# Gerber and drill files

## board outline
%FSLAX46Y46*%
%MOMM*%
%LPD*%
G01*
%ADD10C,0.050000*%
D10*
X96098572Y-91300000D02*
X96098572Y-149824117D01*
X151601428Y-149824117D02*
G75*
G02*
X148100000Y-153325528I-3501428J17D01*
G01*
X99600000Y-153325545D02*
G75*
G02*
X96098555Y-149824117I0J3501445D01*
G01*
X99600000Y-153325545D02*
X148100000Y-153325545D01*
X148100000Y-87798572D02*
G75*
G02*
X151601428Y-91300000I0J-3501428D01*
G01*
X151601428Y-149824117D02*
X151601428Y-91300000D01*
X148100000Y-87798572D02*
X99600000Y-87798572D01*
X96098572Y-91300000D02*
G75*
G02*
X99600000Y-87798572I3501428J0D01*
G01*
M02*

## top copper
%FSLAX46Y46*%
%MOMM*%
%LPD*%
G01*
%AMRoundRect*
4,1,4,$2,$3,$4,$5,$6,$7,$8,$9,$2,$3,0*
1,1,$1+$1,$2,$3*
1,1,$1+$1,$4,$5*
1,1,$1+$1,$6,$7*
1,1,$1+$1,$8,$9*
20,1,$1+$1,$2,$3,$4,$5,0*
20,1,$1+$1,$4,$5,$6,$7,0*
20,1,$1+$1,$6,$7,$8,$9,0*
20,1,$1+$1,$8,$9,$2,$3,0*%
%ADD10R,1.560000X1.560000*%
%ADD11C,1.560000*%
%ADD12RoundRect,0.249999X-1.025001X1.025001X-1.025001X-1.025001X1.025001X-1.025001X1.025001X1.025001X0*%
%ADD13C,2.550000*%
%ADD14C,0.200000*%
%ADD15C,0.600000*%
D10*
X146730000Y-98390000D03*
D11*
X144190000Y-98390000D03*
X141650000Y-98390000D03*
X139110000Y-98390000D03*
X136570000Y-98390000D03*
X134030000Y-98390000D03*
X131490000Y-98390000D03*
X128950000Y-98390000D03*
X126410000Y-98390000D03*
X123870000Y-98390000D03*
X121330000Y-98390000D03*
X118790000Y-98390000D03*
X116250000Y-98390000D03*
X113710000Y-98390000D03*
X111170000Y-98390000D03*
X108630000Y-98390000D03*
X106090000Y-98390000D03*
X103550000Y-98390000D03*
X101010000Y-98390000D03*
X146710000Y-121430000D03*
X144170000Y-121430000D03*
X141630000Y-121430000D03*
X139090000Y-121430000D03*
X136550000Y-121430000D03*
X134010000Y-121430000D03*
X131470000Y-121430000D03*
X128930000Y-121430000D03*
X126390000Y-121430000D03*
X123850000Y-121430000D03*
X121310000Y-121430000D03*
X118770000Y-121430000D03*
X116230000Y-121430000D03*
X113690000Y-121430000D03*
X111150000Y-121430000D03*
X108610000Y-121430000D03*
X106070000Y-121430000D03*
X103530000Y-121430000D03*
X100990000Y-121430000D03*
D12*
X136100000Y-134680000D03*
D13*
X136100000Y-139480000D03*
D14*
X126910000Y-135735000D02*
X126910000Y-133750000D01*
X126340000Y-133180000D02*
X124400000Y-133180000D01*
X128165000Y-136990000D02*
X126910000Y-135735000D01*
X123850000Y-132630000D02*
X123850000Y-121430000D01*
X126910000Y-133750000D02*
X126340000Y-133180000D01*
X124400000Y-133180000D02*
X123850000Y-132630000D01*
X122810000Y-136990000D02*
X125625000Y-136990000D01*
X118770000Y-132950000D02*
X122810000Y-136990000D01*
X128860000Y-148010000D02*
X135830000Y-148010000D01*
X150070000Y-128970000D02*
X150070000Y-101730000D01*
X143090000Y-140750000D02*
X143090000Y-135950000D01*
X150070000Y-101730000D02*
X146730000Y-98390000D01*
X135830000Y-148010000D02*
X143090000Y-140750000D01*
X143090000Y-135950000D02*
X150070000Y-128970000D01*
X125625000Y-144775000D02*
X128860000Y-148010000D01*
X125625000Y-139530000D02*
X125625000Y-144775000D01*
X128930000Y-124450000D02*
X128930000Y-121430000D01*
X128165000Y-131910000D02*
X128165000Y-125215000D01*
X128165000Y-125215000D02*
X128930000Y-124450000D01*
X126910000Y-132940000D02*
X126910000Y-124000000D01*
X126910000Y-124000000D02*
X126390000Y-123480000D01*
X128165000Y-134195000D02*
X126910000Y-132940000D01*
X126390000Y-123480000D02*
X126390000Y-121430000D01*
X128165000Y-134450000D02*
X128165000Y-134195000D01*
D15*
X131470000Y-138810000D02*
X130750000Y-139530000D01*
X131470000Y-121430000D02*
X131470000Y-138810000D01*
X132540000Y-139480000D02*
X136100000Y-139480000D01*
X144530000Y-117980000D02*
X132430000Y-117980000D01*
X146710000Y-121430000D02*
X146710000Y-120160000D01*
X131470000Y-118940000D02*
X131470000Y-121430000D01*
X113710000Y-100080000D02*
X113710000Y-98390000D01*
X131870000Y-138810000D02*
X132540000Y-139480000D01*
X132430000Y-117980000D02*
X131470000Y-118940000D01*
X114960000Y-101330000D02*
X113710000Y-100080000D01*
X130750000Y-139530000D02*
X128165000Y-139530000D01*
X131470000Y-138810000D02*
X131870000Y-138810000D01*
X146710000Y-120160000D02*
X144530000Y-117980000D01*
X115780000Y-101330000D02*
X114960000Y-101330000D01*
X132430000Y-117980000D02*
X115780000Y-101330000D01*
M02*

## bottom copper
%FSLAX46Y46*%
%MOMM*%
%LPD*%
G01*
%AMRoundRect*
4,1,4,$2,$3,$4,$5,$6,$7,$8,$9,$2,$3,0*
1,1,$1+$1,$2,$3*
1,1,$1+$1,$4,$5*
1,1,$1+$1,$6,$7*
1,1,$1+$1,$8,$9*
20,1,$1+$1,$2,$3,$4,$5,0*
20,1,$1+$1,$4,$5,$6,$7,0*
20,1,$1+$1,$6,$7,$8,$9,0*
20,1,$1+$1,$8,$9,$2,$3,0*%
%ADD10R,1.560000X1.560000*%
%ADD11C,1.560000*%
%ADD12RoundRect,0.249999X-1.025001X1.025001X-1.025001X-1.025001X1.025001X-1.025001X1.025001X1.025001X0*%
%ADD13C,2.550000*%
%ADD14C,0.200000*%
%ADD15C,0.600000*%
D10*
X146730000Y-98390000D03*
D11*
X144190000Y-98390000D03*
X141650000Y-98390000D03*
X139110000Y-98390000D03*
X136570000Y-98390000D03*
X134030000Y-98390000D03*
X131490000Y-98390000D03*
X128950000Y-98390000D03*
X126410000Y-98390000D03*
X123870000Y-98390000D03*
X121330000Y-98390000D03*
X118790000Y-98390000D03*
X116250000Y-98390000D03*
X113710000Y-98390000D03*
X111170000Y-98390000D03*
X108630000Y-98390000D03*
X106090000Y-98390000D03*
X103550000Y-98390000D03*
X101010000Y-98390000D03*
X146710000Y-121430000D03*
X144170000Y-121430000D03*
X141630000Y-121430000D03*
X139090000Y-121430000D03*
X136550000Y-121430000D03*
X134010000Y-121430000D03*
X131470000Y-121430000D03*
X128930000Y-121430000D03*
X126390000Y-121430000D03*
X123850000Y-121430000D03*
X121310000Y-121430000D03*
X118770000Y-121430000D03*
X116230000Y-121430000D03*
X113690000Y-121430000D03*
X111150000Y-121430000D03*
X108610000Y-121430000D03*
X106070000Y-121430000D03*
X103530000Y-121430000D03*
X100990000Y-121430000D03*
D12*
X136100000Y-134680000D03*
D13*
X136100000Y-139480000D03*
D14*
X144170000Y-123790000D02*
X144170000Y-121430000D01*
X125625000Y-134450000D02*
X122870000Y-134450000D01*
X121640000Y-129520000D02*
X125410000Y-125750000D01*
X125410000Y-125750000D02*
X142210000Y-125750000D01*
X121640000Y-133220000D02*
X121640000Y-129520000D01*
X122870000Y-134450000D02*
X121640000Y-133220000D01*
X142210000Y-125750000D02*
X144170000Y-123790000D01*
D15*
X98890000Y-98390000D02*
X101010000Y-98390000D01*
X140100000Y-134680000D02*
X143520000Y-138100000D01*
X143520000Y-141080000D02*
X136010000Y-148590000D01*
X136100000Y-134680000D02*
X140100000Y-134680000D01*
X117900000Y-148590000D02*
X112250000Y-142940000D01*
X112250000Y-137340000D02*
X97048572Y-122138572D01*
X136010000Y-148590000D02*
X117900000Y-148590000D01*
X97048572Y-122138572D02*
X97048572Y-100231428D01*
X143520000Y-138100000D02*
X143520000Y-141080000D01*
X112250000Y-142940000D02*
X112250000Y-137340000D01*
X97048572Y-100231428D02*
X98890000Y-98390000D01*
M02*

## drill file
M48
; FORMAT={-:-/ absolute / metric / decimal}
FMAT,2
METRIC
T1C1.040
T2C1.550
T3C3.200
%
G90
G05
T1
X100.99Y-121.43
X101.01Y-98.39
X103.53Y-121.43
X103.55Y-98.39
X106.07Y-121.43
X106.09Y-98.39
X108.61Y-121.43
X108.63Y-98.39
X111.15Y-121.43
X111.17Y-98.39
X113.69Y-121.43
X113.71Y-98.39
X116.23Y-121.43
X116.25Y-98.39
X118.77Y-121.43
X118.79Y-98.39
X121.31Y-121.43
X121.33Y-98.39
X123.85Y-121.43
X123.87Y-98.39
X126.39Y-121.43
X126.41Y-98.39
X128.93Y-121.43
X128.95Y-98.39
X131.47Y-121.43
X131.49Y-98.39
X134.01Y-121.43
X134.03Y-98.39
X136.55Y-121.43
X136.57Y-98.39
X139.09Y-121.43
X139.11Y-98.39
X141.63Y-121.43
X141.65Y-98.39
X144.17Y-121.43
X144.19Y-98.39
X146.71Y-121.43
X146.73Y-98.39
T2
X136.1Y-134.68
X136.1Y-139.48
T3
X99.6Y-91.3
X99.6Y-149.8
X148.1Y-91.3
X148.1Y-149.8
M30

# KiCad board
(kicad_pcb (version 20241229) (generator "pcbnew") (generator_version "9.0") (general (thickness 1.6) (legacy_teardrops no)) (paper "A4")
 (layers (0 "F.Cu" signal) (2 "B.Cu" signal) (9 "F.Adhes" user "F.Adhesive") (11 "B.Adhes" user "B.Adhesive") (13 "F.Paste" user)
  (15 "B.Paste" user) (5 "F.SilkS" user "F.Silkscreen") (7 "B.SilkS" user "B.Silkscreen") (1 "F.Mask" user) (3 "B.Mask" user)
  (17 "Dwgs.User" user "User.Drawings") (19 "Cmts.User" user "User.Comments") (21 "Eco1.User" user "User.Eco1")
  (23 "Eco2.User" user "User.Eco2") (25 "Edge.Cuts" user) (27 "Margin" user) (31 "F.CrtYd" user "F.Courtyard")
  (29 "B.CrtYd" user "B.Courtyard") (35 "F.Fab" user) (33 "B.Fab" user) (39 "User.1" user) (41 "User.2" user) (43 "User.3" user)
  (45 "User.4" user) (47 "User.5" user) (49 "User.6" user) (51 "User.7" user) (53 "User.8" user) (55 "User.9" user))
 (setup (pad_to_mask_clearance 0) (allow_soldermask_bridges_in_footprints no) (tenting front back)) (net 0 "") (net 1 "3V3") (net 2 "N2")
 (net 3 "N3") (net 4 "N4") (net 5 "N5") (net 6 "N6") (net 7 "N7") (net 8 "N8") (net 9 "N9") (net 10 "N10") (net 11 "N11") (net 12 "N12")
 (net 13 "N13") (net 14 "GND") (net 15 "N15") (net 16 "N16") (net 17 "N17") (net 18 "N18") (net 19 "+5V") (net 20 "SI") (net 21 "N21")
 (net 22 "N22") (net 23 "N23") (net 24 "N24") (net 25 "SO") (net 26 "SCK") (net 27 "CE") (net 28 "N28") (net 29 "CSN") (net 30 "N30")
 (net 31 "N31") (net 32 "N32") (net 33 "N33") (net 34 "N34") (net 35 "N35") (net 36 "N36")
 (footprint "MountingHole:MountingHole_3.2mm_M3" (layer "F.Cu") (at 148.1 91.3 180)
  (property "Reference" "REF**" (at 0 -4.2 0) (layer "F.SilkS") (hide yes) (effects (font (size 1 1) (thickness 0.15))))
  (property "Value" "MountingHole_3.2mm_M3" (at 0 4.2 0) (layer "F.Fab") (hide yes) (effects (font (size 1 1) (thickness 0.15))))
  (pad "" np_thru_hole circle (at 0 0 180) (size 3.2 3.2) (drill 3.2) (layers "*.Cu" "*.Mask")))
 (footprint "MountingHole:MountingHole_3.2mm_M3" (layer "F.Cu") (at 99.6 91.3 180)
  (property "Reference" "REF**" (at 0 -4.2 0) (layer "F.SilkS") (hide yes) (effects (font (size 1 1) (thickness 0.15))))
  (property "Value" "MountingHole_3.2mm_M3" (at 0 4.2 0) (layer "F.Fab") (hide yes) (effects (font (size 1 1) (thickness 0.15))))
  (pad "" np_thru_hole circle (at 0 0 180) (size 3.2 3.2) (drill 3.2) (layers "*.Cu" "*.Mask")))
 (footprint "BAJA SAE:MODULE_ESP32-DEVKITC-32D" (layer "F.Cu") (at 127.8 110.15 -90)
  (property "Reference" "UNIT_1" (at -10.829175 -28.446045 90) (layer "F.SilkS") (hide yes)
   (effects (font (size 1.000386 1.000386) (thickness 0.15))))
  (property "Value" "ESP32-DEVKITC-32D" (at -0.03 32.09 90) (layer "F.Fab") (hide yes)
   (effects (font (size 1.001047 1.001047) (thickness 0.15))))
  (pad "J2-1" thru_hole rect (at -11.76 -18.93 270) (size 1.56 1.56) (drill 1.04) (layers "*.Cu" "*.Mask") (remove_unused_layers no)
   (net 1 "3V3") (solder_mask_margin 0.102))
  (pad "J2-2" thru_hole circle (at -11.76 -16.39 270) (size 1.56 1.56) (drill 1.04) (layers "*.Cu" "*.Mask") (remove_unused_layers no)
   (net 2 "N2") (solder_mask_margin 0.102))
  (pad "J2-3" thru_hole circle (at -11.76 -13.85 270) (size 1.56 1.56) (drill 1.04) (layers "*.Cu" "*.Mask") (remove_unused_layers no)
   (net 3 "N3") (solder_mask_margin 0.102))
  (pad "J2-4" thru_hole circle (at -11.76 -11.31 270) (size 1.56 1.56) (drill 1.04) (layers "*.Cu" "*.Mask") (remove_unused_layers no)
   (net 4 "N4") (solder_mask_margin 0.102))
  (pad "J2-5" thru_hole circle (at -11.76 -8.77 270) (size 1.56 1.56) (drill 1.04) (layers "*.Cu" "*.Mask") (remove_unused_layers no)
   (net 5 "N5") (solder_mask_margin 0.102))
  (pad "J2-6" thru_hole circle (at -11.76 -6.23 270) (size 1.56 1.56) (drill 1.04) (layers "*.Cu" "*.Mask") (remove_unused_layers no)
   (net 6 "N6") (solder_mask_margin 0.102))
  (pad "J2-7" thru_hole circle (at -11.76 -3.69 270) (size 1.56 1.56) (drill 1.04) (layers "*.Cu" "*.Mask") (remove_unused_layers no)
   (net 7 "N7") (solder_mask_margin 0.102))
  (pad "J2-8" thru_hole circle (at -11.76 -1.15 270) (size 1.56 1.56) (drill 1.04) (layers "*.Cu" "*.Mask") (remove_unused_layers no)
   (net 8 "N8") (solder_mask_margin 0.102))
  (pad "J2-9" thru_hole circle (at -11.76 1.39 270) (size 1.56 1.56) (drill 1.04) (layers "*.Cu" "*.Mask") (remove_unused_layers no)
   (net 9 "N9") (solder_mask_margin 0.102))
  (pad "J2-10" thru_hole circle (at -11.76 3.93 270) (size 1.56 1.56) (drill 1.04) (layers "*.Cu" "*.Mask") (remove_unused_layers no)
   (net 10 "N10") (solder_mask_margin 0.102))
  (pad "J2-11" thru_hole circle (at -11.76 6.47 270) (size 1.56 1.56) (drill 1.04) (layers "*.Cu" "*.Mask") (remove_unused_layers no)
   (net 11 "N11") (solder_mask_margin 0.102))
  (pad "J2-12" thru_hole circle (at -11.76 9.01 270) (size 1.56 1.56) (drill 1.04) (layers "*.Cu" "*.Mask") (remove_unused_layers no)
   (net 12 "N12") (solder_mask_margin 0.102))
  (pad "J2-13" thru_hole circle (at -11.76 11.55 270) (size 1.56 1.56) (drill 1.04) (layers "*.Cu" "*.Mask") (remove_unused_layers no)
   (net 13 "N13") (solder_mask_margin 0.102))
  (pad "J2-14" thru_hole circle (at -11.76 14.09 270) (size 1.56 1.56) (drill 1.04) (layers "*.Cu" "*.Mask") (remove_unused_layers no)
   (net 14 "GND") (solder_mask_margin 0.102))
  (pad "J2-15" thru_hole circle (at -11.76 16.63 270) (size 1.56 1.56) (drill 1.04) (layers "*.Cu" "*.Mask") (remove_unused_layers no)
   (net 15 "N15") (solder_mask_margin 0.102))
  (pad "J2-16" thru_hole circle (at -11.76 19.17 270) (size 1.56 1.56) (drill 1.04) (layers "*.Cu" "*.Mask") (remove_unused_layers no)
   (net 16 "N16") (solder_mask_margin 0.102))
  (pad "J2-17" thru_hole circle (at -11.76 21.71 270) (size 1.56 1.56) (drill 1.04) (layers "*.Cu" "*.Mask") (remove_unused_layers no)
   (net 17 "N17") (solder_mask_margin 0.102))
  (pad "J2-18" thru_hole circle (at -11.76 24.25 270) (size 1.56 1.56) (drill 1.04) (layers "*.Cu" "*.Mask") (remove_unused_layers no)
   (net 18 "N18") (solder_mask_margin 0.102))
  (pad "J2-19" thru_hole circle (at -11.76 26.79 270) (size 1.56 1.56) (drill 1.04) (layers "*.Cu" "*.Mask") (remove_unused_layers no)
   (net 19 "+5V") (solder_mask_margin 0.102))
  (pad "J3-1" thru_hole circle (at 11.28 -18.91 270) (size 1.56 1.56) (drill 1.04) (layers "*.Cu" "*.Mask") (remove_unused_layers no)
   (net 14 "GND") (solder_mask_margin 0.102))
  (pad "J3-2" thru_hole circle (at 11.28 -16.37 270) (size 1.56 1.56) (drill 1.04) (layers "*.Cu" "*.Mask") (remove_unused_layers no)
   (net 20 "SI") (solder_mask_margin 0.102))
  (pad "J3-3" thru_hole circle (at 11.28 -13.83 270) (size 1.56 1.56) (drill 1.04) (layers "*.Cu" "*.Mask") (remove_unused_layers no)
   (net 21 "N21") (solder_mask_margin 0.102))
  (pad "J3-4" thru_hole circle (at 11.28 -11.29 270) (size 1.56 1.56) (drill 1.04) (layers "*.Cu" "*.Mask") (remove_unused_layers no)
   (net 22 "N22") (solder_mask_margin 0.102))
  (pad "J3-5" thru_hole circle (at 11.28 -8.75 270) (size 1.56 1.56) (drill 1.04) (layers "*.Cu" "*.Mask") (remove_unused_layers no)
   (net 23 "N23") (solder_mask_margin 0.102))
  (pad "J3-6" thru_hole circle (at 11.28 -6.21 270) (size 1.56 1.56) (drill 1.04) (layers "*.Cu" "*.Mask") (remove_unused_layers no)
   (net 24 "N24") (solder_mask_margin 0.102))
  (pad "J3-7" thru_hole circle (at 11.28 -3.67 270) (size 1.56 1.56) (drill 1.04) (layers "*.Cu" "*.Mask") (remove_unused_layers no)
   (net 14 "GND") (solder_mask_margin 0.102))
  (pad "J3-8" thru_hole circle (at 11.28 -1.13 270) (size 1.56 1.56) (drill 1.04) (layers "*.Cu" "*.Mask") (remove_unused_layers no)
   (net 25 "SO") (solder_mask_margin 0.102))
  (pad "J3-9" thru_hole circle (at 11.28 1.41 270) (size 1.56 1.56) (drill 1.04) (layers "*.Cu" "*.Mask") (remove_unused_layers no)
   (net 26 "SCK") (solder_mask_margin 0.102))
  (pad "J3-10" thru_hole circle (at 11.28 3.95 270) (size 1.56 1.56) (drill 1.04) (layers "*.Cu" "*.Mask") (remove_unused_layers no)
   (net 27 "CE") (solder_mask_margin 0.102))
  (pad "J3-11" thru_hole circle (at 11.28 6.49 270) (size 1.56 1.56) (drill 1.04) (layers "*.Cu" "*.Mask") (remove_unused_layers no)
   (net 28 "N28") (solder_mask_margin 0.102))
  (pad "J3-12" thru_hole circle (at 11.28 9.03 270) (size 1.56 1.56) (drill 1.04) (layers "*.Cu" "*.Mask") (remove_unused_layers no)
   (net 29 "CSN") (solder_mask_margin 0.102))
  (pad "J3-13" thru_hole circle (at 11.28 11.57 270) (size 1.56 1.56) (drill 1.04) (layers "*.Cu" "*.Mask") (remove_unused_layers no)
   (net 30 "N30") (solder_mask_margin 0.102))
  (pad "J3-14" thru_hole circle (at 11.28 14.11 270) (size 1.56 1.56) (drill 1.04) (layers "*.Cu" "*.Mask") (remove_unused_layers no)
   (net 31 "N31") (solder_mask_margin 0.102))
  (pad "J3-15" thru_hole circle (at 11.28 16.65 270) (size 1.56 1.56) (drill 1.04) (layers "*.Cu" "*.Mask") (remove_unused_layers no)
   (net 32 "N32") (solder_mask_margin 0.102))
  (pad "J3-16" thru_hole circle (at 11.28 19.19 270) (size 1.56 1.56) (drill 1.04) (layers "*.Cu" "*.Mask") (remove_unused_layers no)
   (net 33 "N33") (solder_mask_margin 0.102))
  (pad "J3-17" thru_hole circle (at 11.28 21.73 270) (size 1.56 1.56) (drill 1.04) (layers "*.Cu" "*.Mask") (remove_unused_layers no)
   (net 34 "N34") (solder_mask_margin 0.102))
  (pad "J3-18" thru_hole circle (at 11.28 24.27 270) (size 1.56 1.56) (drill 1.04) (layers "*.Cu" "*.Mask") (remove_unused_layers no)
   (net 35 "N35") (solder_mask_margin 0.102))
  (pad "J3-19" thru_hole circle (at 11.28 26.81 270) (size 1.56 1.56) (drill 1.04) (layers "*.Cu" "*.Mask") (remove_unused_layers no)
   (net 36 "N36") (solder_mask_margin 0.102)))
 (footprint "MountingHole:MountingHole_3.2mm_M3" (layer "F.Cu") (at 99.6 149.8)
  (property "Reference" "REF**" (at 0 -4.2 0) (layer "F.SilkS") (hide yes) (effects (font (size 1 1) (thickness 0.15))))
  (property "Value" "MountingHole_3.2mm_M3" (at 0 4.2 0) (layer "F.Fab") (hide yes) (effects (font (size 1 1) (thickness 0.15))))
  (pad "" np_thru_hole circle (at 0 0) (size 3.2 3.2) (drill 3.2) (layers "*.Cu" "*.Mask")))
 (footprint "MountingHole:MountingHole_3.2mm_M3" (layer "F.Cu") (at 148.1 149.8)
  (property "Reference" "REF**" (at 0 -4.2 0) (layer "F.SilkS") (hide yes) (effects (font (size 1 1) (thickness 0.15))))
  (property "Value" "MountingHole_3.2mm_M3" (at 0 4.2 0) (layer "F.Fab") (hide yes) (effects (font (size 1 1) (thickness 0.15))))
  (pad "" np_thru_hole circle (at 0 0) (size 3.2 3.2) (drill 3.2) (layers "*.Cu" "*.Mask")))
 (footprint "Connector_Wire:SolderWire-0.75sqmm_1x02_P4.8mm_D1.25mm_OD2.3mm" (layer "F.Cu") (at 136.1 134.68 -90)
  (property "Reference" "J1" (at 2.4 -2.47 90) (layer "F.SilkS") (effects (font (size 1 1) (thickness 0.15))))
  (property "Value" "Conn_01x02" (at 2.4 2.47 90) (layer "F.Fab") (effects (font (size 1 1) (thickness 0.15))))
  (pad "1" thru_hole roundrect (at 0 0 270) (size 2.55 2.55) (drill 1.55) (layers "*.Cu" "*.Mask") (remove_unused_layers no)
   (roundrect_rratio 0.098039) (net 19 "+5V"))
  (pad "2" thru_hole circle (at 4.8 0 270) (size 2.55 2.55) (drill 1.55) (layers "*.Cu" "*.Mask") (remove_unused_layers no) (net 14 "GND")))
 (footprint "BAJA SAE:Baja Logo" (layer "B.Cu") (at 124.22 104.45 180)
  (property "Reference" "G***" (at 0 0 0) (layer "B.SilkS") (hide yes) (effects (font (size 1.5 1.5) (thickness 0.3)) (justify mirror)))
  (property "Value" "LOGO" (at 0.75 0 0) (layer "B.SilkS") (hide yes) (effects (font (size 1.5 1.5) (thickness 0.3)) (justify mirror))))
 (gr_line (start 96.098572 91.3) (end 96.098572 149.824117) (stroke (width 0.05) (type default)) (layer "Edge.Cuts"))
 (gr_arc (start 151.601428 149.824117) (mid 150.575883 152.3) (end 148.1 153.325545) (stroke (width 0.05) (type default)) (locked yes)
  (layer "Edge.Cuts"))
 (gr_arc (start 99.6 153.325545) (mid 97.124117 152.3) (end 96.098572 149.824117) (stroke (width 0.05) (type default)) (layer "Edge.Cuts"))
 (gr_line (start 99.6 153.325545) (end 148.1 153.325545) (stroke (width 0.05) (type default)) (layer "Edge.Cuts"))
 (gr_arc (start 148.1 87.798572) (mid 150.575883 88.824117) (end 151.601428 91.3) (stroke (width 0.05) (type default)) (locked yes)
  (layer "Edge.Cuts"))
 (gr_line (start 151.601428 149.824117) (end 151.601428 91.3) (stroke (width 0.05) (type default)) (layer "Edge.Cuts"))
 (gr_line (start 148.1 87.798572) (end 99.6 87.798572) (stroke (width 0.05) (type default)) (layer "Edge.Cuts"))
 (gr_arc (start 96.098572 91.3) (mid 97.124117 88.824117) (end 99.6 87.798572) (stroke (width 0.05) (type default)) (locked yes)
  (layer "Edge.Cuts"))
 (segment (start 126.91 135.735) (end 126.91 133.75) (width 0.2) (layer "F.Cu") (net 27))
 (segment (start 126.34 133.18) (end 124.4 133.18) (width 0.2) (layer "F.Cu") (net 27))
 (segment (start 128.165 136.99) (end 126.91 135.735) (width 0.2) (layer "F.Cu") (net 27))
 (segment (start 123.85 132.63) (end 123.85 121.43) (width 0.2) (layer "F.Cu") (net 27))
 (segment (start 126.91 133.75) (end 126.34 133.18) (width 0.2) (layer "F.Cu") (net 27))
 (segment (start 124.4 133.18) (end 123.85 132.63) (width 0.2) (layer "F.Cu") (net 27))
 (segment (start 122.81 136.99) (end 125.625 136.99) (width 0.2) (layer "F.Cu") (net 29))
 (segment (start 118.77 132.95) (end 122.81 136.99) (width 0.2) (layer "F.Cu") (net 29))
 (segment (start 128.86 148.01) (end 135.83 148.01) (width 0.2) (layer "F.Cu") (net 1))
 (segment (start 150.07 128.97) (end 150.07 101.73) (width 0.2) (layer "F.Cu") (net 1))
 (segment (start 143.09 140.75) (end 143.09 135.95) (width 0.2) (layer "F.Cu") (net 1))
 (segment (start 150.07 101.73) (end 146.73 98.39) (width 0.2) (layer "F.Cu") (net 1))
 (segment (start 135.83 148.01) (end 143.09 140.75) (width 0.2) (layer "F.Cu") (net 1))
 (segment (start 143.09 135.95) (end 150.07 128.97) (width 0.2) (layer "F.Cu") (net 1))
 (segment (start 125.625 144.775) (end 128.86 148.01) (width 0.2) (layer "F.Cu") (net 1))
 (segment (start 125.625 139.53) (end 125.625 144.775) (width 0.2) (layer "F.Cu") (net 1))
 (segment (start 128.93 124.45) (end 128.93 121.43) (width 0.2) (layer "F.Cu") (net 25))
 (segment (start 128.165 131.91) (end 128.165 125.215) (width 0.2) (layer "F.Cu") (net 25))
 (segment (start 128.165 125.215) (end 128.93 124.45) (width 0.2) (layer "F.Cu") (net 25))
 (segment (start 126.91 132.94) (end 126.91 124) (width 0.2) (layer "F.Cu") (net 26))
 (segment (start 126.91 124) (end 126.39 123.48) (width 0.2) (layer "F.Cu") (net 26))
 (segment (start 128.165 134.195) (end 126.91 132.94) (width 0.2) (layer "F.Cu") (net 26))
 (segment (start 126.39 123.48) (end 126.39 121.43) (width 0.2) (layer "F.Cu") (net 26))
 (segment (start 128.165 134.45) (end 128.165 134.195) (width 0.2) (layer "F.Cu") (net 26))
 (segment (start 144.17 123.79) (end 144.17 121.43) (width 0.2) (layer "B.Cu") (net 20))
 (segment (start 125.625 134.45) (end 122.87 134.45) (width 0.2) (layer "B.Cu") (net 20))
 (segment (start 121.64 129.52) (end 125.41 125.75) (width 0.2) (layer "B.Cu") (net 20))
 (segment (start 125.41 125.75) (end 142.21 125.75) (width 0.2) (layer "B.Cu") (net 20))
 (segment (start 121.64 133.22) (end 121.64 129.52) (width 0.2) (layer "B.Cu") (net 20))
 (segment (start 122.87 134.45) (end 121.64 133.22) (width 0.2) (layer "B.Cu") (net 20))
 (segment (start 142.21 125.75) (end 144.17 123.79) (width 0.2) (layer "B.Cu") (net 20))
 (segment (start 131.47 138.81) (end 130.75 139.53) (width 0.6) (layer "F.Cu") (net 14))
 (segment (start 131.47 121.43) (end 131.47 138.81) (width 0.6) (layer "F.Cu") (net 14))
 (segment (start 132.54 139.48) (end 136.1 139.48) (width 0.6) (layer "F.Cu") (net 14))
 (segment (start 144.53 117.98) (end 132.43 117.98) (width 0.6) (layer "F.Cu") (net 14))
 (segment (start 146.71 121.43) (end 146.71 120.16) (width 0.6) (layer "F.Cu") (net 14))
 (segment (start 131.47 118.94) (end 131.47 121.43) (width 0.6) (layer "F.Cu") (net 14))
 (segment (start 113.71 100.08) (end 113.71 98.39) (width 0.6) (layer "F.Cu") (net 14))
 (segment (start 131.87 138.81) (end 132.54 139.48) (width 0.6) (layer "F.Cu") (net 14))
 (segment (start 132.43 117.98) (end 131.47 118.94) (width 0.6) (layer "F.Cu") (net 14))
 (segment (start 114.96 101.33) (end 113.71 100.08) (width 0.6) (layer "F.Cu") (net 14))
 (segment (start 130.75 139.53) (end 128.165 139.53) (width 0.6) (layer "F.Cu") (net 14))
 (segment (start 131.47 138.81) (end 131.87 138.81) (width 0.6) (layer "F.Cu") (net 14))
 (segment (start 146.71 120.16) (end 144.53 117.98) (width 0.6) (layer "F.Cu") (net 14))
 (segment (start 115.78 101.33) (end 114.96 101.33) (width 0.6) (layer "F.Cu") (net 14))
 (segment (start 132.43 117.98) (end 115.78 101.33) (width 0.6) (layer "F.Cu") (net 14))
 (segment (start 98.89 98.39) (end 101.01 98.39) (width 0.6) (layer "B.Cu") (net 19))
 (segment (start 140.1 134.68) (end 143.52 138.1) (width 0.6) (layer "B.Cu") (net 19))
 (segment (start 143.52 141.08) (end 136.01 148.59) (width 0.6) (layer "B.Cu") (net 19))
 (segment (start 136.1 134.68) (end 140.1 134.68) (width 0.6) (layer "B.Cu") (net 19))
 (segment (start 117.9 148.59) (end 112.25 142.94) (width 0.6) (layer "B.Cu") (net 19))
 (segment (start 112.25 137.34) (end 97.048572 122.138572) (width 0.6) (layer "B.Cu") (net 19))
 (segment (start 136.01 148.59) (end 117.9 148.59) (width 0.6) (layer "B.Cu") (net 19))
 (segment (start 97.048572 122.138572) (end 97.048572 100.231428) (width 0.6) (layer "B.Cu") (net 19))
 (segment (start 143.52 138.1) (end 143.52 141.08) (width 0.6) (layer "B.Cu") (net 19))
 (segment (start 112.25 142.94) (end 112.25 137.34) (width 0.6) (layer "B.Cu") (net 19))
 (segment (start 97.048572 100.231428) (end 98.89 98.39) (width 0.6) (layer "B.Cu") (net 19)))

